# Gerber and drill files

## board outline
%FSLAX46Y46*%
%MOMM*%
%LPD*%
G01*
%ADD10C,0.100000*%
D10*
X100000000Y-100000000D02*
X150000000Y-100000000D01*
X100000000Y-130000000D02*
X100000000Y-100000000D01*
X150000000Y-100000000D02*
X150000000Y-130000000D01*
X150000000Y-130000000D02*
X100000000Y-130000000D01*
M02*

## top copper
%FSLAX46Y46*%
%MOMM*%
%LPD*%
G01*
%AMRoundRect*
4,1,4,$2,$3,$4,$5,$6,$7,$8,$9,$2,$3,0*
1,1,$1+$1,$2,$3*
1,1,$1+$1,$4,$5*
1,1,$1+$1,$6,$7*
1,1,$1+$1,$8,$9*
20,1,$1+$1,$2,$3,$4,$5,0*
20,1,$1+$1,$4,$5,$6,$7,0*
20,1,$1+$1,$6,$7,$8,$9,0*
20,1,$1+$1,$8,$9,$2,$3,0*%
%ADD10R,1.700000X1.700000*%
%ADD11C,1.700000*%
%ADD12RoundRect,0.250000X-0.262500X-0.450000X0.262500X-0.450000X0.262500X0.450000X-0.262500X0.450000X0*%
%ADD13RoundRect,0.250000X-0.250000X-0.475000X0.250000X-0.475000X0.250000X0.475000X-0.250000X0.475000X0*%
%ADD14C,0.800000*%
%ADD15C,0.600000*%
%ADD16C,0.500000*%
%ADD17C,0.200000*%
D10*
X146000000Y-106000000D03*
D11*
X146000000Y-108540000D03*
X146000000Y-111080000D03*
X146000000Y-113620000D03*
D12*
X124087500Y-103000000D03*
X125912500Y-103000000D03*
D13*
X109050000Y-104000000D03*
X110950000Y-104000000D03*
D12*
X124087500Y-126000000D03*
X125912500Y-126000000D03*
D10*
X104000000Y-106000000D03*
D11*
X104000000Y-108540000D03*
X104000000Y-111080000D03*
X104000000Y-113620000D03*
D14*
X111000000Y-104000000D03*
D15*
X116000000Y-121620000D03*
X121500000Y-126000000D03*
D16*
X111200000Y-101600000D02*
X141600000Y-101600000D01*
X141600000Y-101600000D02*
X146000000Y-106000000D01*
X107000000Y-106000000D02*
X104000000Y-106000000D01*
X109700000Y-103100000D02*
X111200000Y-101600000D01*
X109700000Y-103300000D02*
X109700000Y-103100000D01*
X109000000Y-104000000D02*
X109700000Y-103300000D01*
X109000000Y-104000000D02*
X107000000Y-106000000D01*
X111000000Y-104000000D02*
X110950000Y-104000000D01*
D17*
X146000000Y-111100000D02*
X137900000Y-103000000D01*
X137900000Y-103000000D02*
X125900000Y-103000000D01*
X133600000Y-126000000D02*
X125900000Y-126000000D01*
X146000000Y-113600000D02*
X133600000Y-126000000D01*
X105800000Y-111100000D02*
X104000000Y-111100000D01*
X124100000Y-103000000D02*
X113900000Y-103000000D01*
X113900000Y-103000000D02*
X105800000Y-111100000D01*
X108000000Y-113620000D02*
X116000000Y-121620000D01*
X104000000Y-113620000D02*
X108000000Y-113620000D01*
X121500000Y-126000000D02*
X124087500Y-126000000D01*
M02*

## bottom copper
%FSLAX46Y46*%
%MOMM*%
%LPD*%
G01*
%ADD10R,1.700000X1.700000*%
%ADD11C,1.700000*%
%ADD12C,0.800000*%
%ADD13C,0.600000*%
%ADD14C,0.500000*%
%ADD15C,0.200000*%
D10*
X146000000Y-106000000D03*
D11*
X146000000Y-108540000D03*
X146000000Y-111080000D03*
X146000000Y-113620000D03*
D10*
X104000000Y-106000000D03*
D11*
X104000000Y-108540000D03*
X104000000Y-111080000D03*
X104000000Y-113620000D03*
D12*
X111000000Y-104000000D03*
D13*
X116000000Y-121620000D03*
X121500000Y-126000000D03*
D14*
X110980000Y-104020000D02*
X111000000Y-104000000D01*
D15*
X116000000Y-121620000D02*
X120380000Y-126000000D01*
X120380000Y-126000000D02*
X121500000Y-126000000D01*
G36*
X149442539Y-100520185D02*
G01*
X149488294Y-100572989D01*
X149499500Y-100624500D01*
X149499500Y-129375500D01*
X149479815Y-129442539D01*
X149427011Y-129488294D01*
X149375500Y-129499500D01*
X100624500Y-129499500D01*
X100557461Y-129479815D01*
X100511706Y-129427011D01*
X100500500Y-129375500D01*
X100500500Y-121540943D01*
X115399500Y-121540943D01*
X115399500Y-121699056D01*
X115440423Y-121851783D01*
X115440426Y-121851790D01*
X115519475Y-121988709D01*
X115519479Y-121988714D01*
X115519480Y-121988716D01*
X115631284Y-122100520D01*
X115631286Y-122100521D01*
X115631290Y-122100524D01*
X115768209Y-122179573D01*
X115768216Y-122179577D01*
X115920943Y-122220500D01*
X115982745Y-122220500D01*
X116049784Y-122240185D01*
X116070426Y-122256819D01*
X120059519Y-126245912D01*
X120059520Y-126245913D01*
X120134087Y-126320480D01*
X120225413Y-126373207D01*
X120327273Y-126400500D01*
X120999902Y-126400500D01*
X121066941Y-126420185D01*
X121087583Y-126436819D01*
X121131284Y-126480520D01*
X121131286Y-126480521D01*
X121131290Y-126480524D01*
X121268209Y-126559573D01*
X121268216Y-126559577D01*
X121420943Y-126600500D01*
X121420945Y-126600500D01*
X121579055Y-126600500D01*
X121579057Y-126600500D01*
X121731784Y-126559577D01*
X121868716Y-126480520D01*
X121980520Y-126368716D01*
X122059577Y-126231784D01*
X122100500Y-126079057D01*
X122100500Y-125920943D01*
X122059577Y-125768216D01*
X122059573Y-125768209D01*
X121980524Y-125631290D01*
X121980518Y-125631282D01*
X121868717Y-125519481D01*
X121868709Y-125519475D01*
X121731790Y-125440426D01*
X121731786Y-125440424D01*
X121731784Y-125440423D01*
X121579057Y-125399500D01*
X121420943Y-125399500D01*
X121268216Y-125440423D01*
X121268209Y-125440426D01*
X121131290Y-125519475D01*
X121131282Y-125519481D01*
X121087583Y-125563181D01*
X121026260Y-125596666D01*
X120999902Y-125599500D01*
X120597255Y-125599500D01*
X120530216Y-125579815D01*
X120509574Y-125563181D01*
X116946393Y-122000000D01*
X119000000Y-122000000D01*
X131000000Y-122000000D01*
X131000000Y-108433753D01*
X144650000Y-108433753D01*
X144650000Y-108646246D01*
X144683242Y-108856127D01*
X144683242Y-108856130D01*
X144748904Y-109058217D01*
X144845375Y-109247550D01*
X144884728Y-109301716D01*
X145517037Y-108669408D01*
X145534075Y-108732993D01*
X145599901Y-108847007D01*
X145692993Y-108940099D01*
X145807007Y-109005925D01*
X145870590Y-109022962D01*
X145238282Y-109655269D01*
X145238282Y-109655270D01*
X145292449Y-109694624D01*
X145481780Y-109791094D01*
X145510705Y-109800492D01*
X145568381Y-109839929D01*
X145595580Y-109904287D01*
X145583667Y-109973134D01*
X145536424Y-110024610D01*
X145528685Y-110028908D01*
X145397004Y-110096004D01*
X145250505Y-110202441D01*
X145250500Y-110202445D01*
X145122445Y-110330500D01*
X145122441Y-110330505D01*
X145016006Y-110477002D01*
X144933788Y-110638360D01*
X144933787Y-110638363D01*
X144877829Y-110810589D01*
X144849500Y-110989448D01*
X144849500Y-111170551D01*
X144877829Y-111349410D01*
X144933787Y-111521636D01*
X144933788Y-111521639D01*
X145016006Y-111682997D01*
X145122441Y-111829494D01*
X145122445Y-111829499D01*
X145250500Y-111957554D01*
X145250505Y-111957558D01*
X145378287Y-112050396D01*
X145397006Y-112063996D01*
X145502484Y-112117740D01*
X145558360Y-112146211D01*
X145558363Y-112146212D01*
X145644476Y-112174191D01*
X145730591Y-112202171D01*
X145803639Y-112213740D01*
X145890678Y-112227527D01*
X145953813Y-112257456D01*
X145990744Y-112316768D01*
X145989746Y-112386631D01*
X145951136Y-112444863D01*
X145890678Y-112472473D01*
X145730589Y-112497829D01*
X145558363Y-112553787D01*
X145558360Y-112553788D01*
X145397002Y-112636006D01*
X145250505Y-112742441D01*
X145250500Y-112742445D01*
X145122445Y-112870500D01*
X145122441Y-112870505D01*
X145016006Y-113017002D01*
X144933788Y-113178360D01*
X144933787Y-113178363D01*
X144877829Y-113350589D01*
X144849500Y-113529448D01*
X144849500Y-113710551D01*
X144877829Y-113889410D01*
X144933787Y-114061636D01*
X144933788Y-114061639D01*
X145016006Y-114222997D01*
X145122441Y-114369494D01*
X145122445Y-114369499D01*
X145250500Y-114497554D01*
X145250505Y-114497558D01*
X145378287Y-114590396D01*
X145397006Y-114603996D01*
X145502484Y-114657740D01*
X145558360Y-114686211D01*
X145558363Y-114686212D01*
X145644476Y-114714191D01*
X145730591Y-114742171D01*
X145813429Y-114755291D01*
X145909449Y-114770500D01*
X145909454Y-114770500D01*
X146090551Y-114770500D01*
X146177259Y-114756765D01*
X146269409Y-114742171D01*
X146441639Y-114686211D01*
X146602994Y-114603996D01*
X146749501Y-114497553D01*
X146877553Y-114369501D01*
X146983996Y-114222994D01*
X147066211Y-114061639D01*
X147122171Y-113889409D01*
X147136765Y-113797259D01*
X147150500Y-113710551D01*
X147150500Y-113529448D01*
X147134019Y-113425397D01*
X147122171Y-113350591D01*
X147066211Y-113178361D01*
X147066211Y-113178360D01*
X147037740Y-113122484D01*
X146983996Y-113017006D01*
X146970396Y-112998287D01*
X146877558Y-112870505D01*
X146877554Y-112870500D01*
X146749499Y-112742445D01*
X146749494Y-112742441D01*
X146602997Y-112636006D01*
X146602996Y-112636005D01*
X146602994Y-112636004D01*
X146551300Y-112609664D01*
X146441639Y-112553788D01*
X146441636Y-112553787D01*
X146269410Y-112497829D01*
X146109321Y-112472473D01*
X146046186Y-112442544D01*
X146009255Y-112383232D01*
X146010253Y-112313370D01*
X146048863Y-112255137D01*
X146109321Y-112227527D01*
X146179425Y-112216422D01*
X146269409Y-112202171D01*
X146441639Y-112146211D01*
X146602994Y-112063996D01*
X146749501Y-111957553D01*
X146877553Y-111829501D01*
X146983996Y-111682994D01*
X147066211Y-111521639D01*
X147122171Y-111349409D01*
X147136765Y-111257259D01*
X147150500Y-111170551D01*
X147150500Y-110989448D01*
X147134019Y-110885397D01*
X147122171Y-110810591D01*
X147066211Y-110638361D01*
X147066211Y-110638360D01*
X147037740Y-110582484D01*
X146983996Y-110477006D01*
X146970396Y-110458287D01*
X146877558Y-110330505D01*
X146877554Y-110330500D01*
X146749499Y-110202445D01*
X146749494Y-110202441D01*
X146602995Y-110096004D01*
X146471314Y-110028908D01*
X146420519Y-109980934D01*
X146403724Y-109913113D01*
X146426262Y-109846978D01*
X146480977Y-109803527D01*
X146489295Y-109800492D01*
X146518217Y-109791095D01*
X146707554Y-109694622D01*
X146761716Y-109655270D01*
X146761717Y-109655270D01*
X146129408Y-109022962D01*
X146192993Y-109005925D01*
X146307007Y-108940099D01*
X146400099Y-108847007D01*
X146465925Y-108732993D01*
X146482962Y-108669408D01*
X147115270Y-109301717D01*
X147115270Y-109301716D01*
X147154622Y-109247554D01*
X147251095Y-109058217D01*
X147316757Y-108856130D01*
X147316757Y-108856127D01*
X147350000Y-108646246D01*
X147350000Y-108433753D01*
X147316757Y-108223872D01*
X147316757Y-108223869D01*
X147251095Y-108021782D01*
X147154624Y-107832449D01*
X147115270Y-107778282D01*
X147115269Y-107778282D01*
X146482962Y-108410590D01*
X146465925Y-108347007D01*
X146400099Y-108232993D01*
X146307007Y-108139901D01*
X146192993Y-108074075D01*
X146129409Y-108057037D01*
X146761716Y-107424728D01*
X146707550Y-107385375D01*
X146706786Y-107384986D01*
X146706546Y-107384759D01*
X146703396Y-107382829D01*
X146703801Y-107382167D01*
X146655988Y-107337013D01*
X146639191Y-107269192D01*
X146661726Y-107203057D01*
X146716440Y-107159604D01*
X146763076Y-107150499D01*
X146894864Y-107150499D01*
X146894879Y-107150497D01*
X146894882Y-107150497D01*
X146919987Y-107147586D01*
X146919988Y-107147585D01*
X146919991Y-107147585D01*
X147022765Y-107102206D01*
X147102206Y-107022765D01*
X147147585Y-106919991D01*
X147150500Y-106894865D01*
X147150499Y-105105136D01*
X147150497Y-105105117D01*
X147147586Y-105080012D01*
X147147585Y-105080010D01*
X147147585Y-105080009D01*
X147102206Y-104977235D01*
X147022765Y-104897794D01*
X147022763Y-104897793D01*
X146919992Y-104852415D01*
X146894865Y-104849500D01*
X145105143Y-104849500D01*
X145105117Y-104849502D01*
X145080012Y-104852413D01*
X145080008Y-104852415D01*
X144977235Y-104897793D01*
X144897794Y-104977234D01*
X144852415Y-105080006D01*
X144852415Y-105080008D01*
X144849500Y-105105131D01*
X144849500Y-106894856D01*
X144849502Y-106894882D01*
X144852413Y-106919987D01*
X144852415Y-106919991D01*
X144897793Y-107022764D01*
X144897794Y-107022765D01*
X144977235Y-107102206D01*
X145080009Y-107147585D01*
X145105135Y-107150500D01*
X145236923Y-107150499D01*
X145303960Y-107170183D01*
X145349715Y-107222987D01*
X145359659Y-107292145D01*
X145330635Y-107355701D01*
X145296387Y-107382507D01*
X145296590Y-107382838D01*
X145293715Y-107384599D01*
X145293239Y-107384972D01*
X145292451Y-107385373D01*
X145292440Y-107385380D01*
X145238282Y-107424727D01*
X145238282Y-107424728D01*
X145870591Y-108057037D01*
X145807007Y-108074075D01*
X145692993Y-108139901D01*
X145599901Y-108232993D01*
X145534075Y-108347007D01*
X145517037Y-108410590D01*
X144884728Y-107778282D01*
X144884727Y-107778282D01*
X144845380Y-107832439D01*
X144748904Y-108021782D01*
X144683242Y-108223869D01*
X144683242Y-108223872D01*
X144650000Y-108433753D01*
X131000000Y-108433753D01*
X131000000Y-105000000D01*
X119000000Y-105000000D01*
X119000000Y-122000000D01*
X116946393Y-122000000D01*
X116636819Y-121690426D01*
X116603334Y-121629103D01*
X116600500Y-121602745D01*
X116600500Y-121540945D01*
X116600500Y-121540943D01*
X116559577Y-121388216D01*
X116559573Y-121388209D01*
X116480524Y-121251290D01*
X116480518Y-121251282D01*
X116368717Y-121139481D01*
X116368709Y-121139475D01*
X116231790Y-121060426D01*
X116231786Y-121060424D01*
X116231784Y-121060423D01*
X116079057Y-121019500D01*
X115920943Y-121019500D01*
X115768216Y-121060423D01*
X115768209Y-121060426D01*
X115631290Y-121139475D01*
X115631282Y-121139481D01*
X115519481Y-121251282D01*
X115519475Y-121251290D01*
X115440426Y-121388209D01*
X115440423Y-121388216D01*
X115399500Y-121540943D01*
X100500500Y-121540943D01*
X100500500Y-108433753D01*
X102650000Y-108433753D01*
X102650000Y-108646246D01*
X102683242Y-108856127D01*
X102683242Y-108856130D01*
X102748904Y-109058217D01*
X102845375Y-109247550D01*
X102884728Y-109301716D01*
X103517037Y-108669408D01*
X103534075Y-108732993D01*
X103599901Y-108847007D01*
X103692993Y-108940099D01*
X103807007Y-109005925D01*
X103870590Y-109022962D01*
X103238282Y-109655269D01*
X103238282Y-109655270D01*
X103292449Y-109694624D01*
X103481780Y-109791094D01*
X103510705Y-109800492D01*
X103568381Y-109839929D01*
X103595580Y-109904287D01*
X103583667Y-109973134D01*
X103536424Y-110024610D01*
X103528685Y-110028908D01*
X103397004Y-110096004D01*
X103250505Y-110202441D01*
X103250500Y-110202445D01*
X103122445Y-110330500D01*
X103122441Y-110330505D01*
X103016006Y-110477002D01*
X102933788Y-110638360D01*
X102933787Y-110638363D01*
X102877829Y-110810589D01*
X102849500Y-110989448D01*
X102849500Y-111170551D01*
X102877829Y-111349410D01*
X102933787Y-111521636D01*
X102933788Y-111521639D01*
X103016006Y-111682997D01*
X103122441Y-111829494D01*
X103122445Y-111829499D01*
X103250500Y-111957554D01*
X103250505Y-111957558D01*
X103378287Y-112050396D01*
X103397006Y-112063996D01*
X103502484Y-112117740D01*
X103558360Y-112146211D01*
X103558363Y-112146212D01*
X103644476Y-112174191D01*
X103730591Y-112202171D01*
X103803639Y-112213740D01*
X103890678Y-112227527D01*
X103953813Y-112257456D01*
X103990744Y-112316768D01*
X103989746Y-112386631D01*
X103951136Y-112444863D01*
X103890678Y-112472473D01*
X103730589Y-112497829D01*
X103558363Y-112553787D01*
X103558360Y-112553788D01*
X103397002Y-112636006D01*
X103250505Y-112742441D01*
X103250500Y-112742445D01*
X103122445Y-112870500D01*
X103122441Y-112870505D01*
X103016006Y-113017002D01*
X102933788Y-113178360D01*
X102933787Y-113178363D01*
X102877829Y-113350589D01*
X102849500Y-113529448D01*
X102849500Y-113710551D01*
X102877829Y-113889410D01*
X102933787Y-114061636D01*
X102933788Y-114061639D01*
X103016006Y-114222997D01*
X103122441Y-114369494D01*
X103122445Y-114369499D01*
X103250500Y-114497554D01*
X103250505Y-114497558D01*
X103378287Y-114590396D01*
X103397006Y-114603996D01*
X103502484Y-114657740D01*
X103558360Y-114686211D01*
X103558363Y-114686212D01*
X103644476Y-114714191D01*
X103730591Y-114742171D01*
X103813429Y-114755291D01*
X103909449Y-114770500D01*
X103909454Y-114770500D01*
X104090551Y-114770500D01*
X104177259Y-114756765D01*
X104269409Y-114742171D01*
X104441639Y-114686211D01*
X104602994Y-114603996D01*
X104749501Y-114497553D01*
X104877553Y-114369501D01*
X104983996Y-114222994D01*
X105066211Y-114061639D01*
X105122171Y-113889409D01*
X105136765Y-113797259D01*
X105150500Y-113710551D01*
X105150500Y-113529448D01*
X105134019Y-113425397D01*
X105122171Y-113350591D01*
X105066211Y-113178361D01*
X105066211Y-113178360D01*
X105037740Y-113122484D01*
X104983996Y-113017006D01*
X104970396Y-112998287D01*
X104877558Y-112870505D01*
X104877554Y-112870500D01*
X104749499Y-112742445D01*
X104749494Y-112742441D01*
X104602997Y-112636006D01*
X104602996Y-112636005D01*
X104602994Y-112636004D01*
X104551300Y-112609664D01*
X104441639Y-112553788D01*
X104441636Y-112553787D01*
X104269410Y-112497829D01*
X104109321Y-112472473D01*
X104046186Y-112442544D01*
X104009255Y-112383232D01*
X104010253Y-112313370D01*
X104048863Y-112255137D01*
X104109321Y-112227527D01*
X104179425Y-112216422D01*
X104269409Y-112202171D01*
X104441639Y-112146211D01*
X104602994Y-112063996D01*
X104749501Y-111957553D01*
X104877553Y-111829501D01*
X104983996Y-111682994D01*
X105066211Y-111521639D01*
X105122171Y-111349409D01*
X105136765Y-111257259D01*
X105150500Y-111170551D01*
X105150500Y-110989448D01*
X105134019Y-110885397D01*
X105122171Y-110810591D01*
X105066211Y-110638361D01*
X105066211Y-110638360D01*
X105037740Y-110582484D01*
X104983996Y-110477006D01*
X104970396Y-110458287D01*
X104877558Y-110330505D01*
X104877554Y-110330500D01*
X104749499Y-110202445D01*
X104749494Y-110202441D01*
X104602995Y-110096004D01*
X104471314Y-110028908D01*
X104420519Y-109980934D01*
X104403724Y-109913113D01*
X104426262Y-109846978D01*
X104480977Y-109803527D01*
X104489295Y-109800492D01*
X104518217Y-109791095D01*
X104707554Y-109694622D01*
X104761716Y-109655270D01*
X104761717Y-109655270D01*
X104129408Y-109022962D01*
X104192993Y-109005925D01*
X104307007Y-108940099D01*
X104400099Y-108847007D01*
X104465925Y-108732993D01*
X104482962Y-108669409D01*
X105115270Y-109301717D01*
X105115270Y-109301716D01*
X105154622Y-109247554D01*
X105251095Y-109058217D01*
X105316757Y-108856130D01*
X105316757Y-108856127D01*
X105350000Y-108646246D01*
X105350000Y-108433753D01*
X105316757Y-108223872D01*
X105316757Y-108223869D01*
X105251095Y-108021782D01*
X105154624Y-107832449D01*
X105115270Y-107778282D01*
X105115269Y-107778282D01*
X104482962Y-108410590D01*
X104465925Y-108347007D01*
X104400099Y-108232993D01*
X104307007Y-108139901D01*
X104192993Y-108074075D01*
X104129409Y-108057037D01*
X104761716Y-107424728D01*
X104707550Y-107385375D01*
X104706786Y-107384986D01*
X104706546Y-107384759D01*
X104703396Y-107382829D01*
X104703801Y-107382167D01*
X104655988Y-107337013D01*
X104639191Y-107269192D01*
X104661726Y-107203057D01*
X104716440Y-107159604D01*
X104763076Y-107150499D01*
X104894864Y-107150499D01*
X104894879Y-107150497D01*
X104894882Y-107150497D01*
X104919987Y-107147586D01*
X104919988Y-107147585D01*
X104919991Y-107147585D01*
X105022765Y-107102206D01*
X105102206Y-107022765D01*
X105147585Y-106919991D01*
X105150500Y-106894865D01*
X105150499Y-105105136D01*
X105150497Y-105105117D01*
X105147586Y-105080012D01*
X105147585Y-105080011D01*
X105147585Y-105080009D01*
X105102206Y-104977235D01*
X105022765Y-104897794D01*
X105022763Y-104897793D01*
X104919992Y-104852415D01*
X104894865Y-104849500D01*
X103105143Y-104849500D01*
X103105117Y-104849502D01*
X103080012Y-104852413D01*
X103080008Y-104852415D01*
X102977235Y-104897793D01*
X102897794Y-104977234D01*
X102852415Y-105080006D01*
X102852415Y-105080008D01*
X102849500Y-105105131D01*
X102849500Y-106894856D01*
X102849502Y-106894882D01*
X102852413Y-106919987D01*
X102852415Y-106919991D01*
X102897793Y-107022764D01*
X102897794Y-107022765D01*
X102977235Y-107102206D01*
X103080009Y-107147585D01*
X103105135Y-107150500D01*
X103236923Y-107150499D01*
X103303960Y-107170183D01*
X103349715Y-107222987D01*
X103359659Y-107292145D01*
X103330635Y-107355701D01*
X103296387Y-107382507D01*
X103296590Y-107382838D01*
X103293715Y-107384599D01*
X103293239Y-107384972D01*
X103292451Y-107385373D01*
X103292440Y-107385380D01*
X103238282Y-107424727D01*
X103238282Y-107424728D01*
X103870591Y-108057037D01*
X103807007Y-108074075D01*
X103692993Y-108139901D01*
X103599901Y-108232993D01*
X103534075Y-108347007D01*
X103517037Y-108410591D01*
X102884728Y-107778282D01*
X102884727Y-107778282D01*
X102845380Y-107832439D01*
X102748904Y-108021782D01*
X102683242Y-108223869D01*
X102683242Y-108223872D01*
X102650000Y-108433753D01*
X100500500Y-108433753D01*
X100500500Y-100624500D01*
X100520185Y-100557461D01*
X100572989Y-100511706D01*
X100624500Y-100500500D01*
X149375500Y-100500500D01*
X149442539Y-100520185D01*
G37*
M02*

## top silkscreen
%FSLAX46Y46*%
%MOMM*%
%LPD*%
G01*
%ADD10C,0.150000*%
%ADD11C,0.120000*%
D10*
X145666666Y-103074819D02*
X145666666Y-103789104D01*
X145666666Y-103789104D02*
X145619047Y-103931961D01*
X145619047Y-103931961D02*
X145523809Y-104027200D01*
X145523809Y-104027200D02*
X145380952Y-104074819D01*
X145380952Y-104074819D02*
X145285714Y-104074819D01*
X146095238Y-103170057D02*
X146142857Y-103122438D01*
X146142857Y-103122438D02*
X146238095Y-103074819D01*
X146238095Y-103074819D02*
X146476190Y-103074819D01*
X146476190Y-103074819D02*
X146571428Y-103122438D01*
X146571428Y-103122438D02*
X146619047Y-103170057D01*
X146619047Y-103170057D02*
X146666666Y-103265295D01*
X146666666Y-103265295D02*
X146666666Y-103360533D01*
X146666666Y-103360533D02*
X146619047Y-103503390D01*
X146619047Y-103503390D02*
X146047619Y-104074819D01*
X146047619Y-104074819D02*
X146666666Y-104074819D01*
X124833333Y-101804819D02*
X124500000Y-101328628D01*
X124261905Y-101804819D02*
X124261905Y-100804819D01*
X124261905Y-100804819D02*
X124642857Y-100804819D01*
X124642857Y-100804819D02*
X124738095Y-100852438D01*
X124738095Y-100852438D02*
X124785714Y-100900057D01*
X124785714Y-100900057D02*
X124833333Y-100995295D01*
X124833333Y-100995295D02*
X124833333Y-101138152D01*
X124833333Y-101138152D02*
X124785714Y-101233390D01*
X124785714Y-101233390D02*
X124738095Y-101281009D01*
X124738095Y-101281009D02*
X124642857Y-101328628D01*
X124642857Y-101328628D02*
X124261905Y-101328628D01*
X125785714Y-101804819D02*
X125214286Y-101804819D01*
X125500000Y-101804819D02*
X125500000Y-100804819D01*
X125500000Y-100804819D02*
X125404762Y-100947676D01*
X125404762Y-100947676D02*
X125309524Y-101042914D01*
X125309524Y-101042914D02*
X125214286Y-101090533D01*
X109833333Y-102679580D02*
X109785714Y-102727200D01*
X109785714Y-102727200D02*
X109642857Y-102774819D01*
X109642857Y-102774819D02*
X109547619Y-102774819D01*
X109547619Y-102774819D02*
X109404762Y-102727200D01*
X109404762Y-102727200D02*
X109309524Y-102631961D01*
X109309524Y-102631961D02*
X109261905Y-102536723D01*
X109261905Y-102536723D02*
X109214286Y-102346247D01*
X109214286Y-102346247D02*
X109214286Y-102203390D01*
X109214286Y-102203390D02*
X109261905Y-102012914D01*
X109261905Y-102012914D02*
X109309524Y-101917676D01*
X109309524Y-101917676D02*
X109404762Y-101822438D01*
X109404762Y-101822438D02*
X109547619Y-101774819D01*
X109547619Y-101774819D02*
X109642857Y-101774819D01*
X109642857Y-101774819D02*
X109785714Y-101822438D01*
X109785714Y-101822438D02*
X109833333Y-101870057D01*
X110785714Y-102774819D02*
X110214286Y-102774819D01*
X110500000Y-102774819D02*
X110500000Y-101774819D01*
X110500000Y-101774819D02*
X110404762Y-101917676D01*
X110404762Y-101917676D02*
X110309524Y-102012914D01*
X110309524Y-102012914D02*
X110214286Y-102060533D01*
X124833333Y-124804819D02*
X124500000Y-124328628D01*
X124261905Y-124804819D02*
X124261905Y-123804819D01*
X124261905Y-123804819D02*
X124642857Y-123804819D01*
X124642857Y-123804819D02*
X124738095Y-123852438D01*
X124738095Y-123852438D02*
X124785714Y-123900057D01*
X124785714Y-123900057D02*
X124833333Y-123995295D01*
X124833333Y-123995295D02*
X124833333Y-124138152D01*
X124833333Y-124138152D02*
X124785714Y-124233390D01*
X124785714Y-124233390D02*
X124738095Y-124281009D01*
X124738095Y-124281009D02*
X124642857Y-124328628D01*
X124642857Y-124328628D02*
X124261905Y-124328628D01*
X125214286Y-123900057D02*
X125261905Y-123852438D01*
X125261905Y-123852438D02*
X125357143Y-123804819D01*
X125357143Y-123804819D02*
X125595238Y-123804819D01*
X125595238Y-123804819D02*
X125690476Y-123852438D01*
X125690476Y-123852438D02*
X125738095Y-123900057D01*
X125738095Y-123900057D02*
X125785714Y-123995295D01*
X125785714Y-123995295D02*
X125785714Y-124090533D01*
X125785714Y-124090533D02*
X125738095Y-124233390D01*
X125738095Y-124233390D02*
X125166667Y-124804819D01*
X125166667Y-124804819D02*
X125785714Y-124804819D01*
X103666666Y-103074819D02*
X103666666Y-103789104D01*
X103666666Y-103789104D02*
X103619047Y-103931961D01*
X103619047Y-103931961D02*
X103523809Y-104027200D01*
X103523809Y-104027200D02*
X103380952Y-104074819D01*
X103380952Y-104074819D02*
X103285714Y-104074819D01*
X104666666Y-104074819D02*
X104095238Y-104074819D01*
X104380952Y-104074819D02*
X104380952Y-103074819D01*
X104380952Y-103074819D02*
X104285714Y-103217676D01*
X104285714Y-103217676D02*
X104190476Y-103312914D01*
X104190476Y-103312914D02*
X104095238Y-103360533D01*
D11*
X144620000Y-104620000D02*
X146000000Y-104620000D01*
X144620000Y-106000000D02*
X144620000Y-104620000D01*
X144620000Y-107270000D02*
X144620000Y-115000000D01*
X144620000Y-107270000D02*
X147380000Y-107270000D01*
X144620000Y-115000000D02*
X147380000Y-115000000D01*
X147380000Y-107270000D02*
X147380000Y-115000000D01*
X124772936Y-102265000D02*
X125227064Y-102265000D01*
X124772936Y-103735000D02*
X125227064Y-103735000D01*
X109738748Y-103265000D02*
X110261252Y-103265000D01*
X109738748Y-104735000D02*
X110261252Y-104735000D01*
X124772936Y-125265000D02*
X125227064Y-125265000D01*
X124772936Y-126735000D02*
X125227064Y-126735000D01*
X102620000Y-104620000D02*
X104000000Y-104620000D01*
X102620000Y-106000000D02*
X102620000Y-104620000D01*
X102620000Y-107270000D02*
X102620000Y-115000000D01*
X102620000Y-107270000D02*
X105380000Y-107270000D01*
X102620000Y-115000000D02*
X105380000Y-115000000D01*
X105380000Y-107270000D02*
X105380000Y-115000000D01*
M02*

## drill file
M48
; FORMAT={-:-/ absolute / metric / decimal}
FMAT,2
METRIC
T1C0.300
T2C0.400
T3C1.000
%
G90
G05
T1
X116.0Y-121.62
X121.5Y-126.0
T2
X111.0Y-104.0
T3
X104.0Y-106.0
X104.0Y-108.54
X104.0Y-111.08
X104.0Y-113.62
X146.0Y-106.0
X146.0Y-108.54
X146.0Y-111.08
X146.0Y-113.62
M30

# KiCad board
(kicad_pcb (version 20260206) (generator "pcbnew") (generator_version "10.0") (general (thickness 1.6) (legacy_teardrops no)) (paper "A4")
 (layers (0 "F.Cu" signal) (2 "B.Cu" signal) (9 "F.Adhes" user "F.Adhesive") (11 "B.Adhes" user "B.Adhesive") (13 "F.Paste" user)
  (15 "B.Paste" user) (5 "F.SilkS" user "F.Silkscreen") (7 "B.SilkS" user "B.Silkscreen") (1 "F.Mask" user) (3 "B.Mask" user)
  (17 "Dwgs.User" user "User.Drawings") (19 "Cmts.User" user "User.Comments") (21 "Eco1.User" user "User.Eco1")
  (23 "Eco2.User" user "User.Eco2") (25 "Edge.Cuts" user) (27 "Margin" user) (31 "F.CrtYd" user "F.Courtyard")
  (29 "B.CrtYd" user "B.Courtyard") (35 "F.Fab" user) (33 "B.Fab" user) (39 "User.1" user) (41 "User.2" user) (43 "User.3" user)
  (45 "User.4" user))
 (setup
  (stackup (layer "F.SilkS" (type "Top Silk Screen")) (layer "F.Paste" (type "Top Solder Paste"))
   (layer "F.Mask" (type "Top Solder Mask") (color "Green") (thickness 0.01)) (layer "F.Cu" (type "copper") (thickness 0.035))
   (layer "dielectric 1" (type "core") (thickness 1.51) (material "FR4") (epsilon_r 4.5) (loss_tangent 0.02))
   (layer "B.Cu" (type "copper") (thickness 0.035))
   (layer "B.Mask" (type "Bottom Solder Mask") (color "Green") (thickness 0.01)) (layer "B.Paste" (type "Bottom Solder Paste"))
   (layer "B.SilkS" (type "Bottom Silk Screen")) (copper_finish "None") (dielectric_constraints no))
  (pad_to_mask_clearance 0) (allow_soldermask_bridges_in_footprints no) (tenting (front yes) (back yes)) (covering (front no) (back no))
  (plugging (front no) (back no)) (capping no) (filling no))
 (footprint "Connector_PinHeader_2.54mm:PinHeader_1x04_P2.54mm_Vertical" (layer "F.Cu") (at 146 106)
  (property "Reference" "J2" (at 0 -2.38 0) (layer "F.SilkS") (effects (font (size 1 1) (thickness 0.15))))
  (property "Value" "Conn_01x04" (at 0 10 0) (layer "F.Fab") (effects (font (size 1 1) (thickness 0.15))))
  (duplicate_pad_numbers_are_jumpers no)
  (fp_line (start -1.38 -1.38) (end 0 -1.38) (stroke (width 0.12) (type solid)) (layer "F.SilkS"))
  (fp_line (start -1.38 0) (end -1.38 -1.38) (stroke (width 0.12) (type solid)) (layer "F.SilkS"))
  (fp_line (start -1.38 1.27) (end -1.38 9) (stroke (width 0.12) (type solid)) (layer "F.SilkS"))
  (fp_line (start -1.38 1.27) (end 1.38 1.27) (stroke (width 0.12) (type solid)) (layer "F.SilkS"))
  (fp_line (start -1.38 9) (end 1.38 9) (stroke (width 0.12) (type solid)) (layer "F.SilkS"))
  (fp_line (start 1.38 1.27) (end 1.38 9) (stroke (width 0.12) (type solid)) (layer "F.SilkS"))
  (pad "1" thru_hole rect (at 0 0) (size 1.7 1.7) (drill 1) (layers "*.Cu" "*.Mask") (remove_unused_layers no) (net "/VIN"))
  (pad "2" thru_hole circle (at 0 2.54) (size 1.7 1.7) (drill 1) (layers "*.Cu" "*.Mask") (remove_unused_layers no) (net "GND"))
  (pad "3" thru_hole circle (at 0 5.08) (size 1.7 1.7) (drill 1) (layers "*.Cu" "*.Mask") (remove_unused_layers no) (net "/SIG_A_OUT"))
  (pad "4" thru_hole circle (at 0 7.62) (size 1.7 1.7) (drill 1) (layers "*.Cu" "*.Mask") (remove_unused_layers no) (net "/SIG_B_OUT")))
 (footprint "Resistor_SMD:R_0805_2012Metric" (layer "F.Cu") (at 125 103)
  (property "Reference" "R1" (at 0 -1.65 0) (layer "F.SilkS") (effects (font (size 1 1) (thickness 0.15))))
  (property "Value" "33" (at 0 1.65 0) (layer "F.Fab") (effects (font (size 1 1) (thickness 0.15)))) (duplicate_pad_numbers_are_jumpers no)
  (fp_line (start -0.227064 -0.735) (end 0.227064 -0.735) (stroke (width 0.12) (type solid)) (layer "F.SilkS"))
  (fp_line (start -0.227064 0.735) (end 0.227064 0.735) (stroke (width 0.12) (type solid)) (layer "F.SilkS"))
  (pad "1" smd roundrect (at -0.9125 0) (size 1.025 1.4) (layers "F.Cu" "F.Mask" "F.Paste") (roundrect_rratio 0.243902) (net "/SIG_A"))
  (pad "2" smd roundrect (at 0.9125 0) (size 1.025 1.4) (layers "F.Cu" "F.Mask" "F.Paste") (roundrect_rratio 0.243902) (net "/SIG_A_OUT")))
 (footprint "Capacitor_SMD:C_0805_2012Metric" (layer "F.Cu") (at 110 104)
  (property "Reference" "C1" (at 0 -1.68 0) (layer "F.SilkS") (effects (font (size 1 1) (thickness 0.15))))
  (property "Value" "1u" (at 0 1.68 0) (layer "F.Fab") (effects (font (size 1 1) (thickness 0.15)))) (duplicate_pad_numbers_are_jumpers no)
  (fp_line (start -0.261252 -0.735) (end 0.261252 -0.735) (stroke (width 0.12) (type solid)) (layer "F.SilkS"))
  (fp_line (start -0.261252 0.735) (end 0.261252 0.735) (stroke (width 0.12) (type solid)) (layer "F.SilkS"))
  (pad "1" smd roundrect (at -0.95 0) (size 1 1.45) (layers "F.Cu" "F.Mask" "F.Paste") (roundrect_rratio 0.25) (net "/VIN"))
  (pad "2" smd roundrect (at 0.95 0) (size 1 1.45) (layers "F.Cu" "F.Mask" "F.Paste") (roundrect_rratio 0.25) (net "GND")))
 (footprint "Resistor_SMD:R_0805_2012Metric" (layer "F.Cu") (at 125 126)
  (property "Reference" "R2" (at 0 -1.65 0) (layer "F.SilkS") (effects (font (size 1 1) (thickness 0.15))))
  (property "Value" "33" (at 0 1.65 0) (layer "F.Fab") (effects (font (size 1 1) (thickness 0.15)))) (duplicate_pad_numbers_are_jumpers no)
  (fp_line (start -0.227064 -0.735) (end 0.227064 -0.735) (stroke (width 0.12) (type solid)) (layer "F.SilkS"))
  (fp_line (start -0.227064 0.735) (end 0.227064 0.735) (stroke (width 0.12) (type solid)) (layer "F.SilkS"))
  (pad "1" smd roundrect (at -0.9125 0) (size 1.025 1.4) (layers "F.Cu" "F.Mask" "F.Paste") (roundrect_rratio 0.243902) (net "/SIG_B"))
  (pad "2" smd roundrect (at 0.9125 0) (size 1.025 1.4) (layers "F.Cu" "F.Mask" "F.Paste") (roundrect_rratio 0.243902) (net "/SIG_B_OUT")))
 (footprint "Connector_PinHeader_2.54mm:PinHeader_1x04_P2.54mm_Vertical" (layer "F.Cu") (at 104 106)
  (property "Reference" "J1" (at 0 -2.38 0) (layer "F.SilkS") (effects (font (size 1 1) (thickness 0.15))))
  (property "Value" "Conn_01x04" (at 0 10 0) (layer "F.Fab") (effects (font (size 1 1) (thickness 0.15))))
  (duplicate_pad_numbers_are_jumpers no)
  (fp_line (start -1.38 -1.38) (end 0 -1.38) (stroke (width 0.12) (type solid)) (layer "F.SilkS"))
  (fp_line (start -1.38 0) (end -1.38 -1.38) (stroke (width 0.12) (type solid)) (layer "F.SilkS"))
  (fp_line (start -1.38 1.27) (end -1.38 9) (stroke (width 0.12) (type solid)) (layer "F.SilkS"))
  (fp_line (start -1.38 1.27) (end 1.38 1.27) (stroke (width 0.12) (type solid)) (layer "F.SilkS"))
  (fp_line (start -1.38 9) (end 1.38 9) (stroke (width 0.12) (type solid)) (layer "F.SilkS"))
  (fp_line (start 1.38 1.27) (end 1.38 9) (stroke (width 0.12) (type solid)) (layer "F.SilkS"))
  (pad "1" thru_hole rect (at 0 0) (size 1.7 1.7) (drill 1) (layers "*.Cu" "*.Mask") (remove_unused_layers no) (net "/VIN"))
  (pad "2" thru_hole circle (at 0 2.54) (size 1.7 1.7) (drill 1) (layers "*.Cu" "*.Mask") (remove_unused_layers no) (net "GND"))
  (pad "3" thru_hole circle (at 0 5.08) (size 1.7 1.7) (drill 1) (layers "*.Cu" "*.Mask") (remove_unused_layers no) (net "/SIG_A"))
  (pad "4" thru_hole circle (at 0 7.62) (size 1.7 1.7) (drill 1) (layers "*.Cu" "*.Mask") (remove_unused_layers no) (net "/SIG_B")))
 (gr_line (start 100 100) (end 150 100) (stroke (width 0.1) (type default)) (layer "Edge.Cuts"))
 (gr_line (start 100 130) (end 100 100) (stroke (width 0.1) (type default)) (layer "Edge.Cuts"))
 (gr_line (start 150 100) (end 150 130) (stroke (width 0.1) (type default)) (layer "Edge.Cuts"))
 (gr_line (start 150 130) (end 100 130) (stroke (width 0.1) (type default)) (layer "Edge.Cuts"))
 (segment (start 111.2 101.6) (end 141.6 101.6) (width 0.5) (layer "F.Cu") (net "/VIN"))
 (segment (start 141.6 101.6) (end 146 106) (width 0.5) (layer "F.Cu") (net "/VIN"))
 (segment (start 107 106) (end 104 106) (width 0.5) (layer "F.Cu") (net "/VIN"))
 (segment (start 109.7 103.1) (end 111.2 101.6) (width 0.5) (layer "F.Cu") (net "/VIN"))
 (segment (start 109.7 103.3) (end 109.7 103.1) (width 0.5) (layer "F.Cu") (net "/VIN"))
 (segment (start 109 104) (end 109.7 103.3) (width 0.5) (layer "F.Cu") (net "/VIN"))
 (segment (start 109 104) (end 107 106) (width 0.5) (layer "F.Cu") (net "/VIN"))
 (segment (start 111 104) (end 110.95 104) (width 0.5) (layer "F.Cu") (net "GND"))
 (via (at 111 104) (size 0.8) (drill 0.4) (layers "F.Cu" "B.Cu") (capping yes) (filling yes) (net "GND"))
 (segment (start 110.98 104.02) (end 111 104) (width 0.5) (layer "B.Cu") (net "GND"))
 (segment (start 146 111.1) (end 137.9 103) (width 0.2) (layer "F.Cu") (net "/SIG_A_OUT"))
 (segment (start 137.9 103) (end 125.9 103) (width 0.2) (layer "F.Cu") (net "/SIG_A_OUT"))
 (segment (start 133.6 126) (end 125.9 126) (width 0.2) (layer "F.Cu") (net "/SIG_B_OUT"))
 (segment (start 146 113.6) (end 133.6 126) (width 0.2) (layer "F.Cu") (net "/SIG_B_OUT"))
 (segment (start 105.8 111.1) (end 104 111.1) (width 0.2) (layer "F.Cu") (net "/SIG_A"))
 (segment (start 124.1 103) (end 113.9 103) (width 0.2) (layer "F.Cu") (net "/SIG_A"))
 (segment (start 113.9 103) (end 105.8 111.1) (width 0.2) (layer "F.Cu") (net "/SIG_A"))
 (segment (start 108 113.62) (end 116 121.62) (width 0.2) (locked yes) (layer "F.Cu") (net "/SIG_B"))
 (segment (start 104 113.62) (end 108 113.62) (width 0.2) (locked yes) (layer "F.Cu") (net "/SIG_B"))
 (segment (start 121.5 126) (end 124.0875 126) (width 0.2) (locked yes) (layer "F.Cu") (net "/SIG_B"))
 (via (at 116 121.62) (size 0.6) (drill 0.3) (layers "F.Cu" "B.Cu") (locked yes) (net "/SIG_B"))
 (via (at 121.5 126) (size 0.6) (drill 0.3) (layers "F.Cu" "B.Cu") (locked yes) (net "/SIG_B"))
 (segment (start 116 121.62) (end 120.38 126) (width 0.2) (locked yes) (layer "B.Cu") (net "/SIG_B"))
 (segment (start 120.38 126) (end 121.5 126) (width 0.2) (locked yes) (layer "B.Cu") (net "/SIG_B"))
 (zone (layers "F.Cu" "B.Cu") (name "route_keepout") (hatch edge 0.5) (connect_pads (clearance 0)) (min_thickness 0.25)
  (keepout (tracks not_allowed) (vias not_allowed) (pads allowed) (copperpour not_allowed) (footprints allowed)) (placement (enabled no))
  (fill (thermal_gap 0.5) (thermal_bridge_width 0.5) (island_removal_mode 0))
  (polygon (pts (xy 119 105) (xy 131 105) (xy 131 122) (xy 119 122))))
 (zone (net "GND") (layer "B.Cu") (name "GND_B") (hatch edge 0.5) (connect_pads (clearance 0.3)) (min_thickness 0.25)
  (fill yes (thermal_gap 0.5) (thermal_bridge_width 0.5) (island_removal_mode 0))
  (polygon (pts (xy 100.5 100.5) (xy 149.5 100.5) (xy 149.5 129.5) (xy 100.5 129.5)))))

